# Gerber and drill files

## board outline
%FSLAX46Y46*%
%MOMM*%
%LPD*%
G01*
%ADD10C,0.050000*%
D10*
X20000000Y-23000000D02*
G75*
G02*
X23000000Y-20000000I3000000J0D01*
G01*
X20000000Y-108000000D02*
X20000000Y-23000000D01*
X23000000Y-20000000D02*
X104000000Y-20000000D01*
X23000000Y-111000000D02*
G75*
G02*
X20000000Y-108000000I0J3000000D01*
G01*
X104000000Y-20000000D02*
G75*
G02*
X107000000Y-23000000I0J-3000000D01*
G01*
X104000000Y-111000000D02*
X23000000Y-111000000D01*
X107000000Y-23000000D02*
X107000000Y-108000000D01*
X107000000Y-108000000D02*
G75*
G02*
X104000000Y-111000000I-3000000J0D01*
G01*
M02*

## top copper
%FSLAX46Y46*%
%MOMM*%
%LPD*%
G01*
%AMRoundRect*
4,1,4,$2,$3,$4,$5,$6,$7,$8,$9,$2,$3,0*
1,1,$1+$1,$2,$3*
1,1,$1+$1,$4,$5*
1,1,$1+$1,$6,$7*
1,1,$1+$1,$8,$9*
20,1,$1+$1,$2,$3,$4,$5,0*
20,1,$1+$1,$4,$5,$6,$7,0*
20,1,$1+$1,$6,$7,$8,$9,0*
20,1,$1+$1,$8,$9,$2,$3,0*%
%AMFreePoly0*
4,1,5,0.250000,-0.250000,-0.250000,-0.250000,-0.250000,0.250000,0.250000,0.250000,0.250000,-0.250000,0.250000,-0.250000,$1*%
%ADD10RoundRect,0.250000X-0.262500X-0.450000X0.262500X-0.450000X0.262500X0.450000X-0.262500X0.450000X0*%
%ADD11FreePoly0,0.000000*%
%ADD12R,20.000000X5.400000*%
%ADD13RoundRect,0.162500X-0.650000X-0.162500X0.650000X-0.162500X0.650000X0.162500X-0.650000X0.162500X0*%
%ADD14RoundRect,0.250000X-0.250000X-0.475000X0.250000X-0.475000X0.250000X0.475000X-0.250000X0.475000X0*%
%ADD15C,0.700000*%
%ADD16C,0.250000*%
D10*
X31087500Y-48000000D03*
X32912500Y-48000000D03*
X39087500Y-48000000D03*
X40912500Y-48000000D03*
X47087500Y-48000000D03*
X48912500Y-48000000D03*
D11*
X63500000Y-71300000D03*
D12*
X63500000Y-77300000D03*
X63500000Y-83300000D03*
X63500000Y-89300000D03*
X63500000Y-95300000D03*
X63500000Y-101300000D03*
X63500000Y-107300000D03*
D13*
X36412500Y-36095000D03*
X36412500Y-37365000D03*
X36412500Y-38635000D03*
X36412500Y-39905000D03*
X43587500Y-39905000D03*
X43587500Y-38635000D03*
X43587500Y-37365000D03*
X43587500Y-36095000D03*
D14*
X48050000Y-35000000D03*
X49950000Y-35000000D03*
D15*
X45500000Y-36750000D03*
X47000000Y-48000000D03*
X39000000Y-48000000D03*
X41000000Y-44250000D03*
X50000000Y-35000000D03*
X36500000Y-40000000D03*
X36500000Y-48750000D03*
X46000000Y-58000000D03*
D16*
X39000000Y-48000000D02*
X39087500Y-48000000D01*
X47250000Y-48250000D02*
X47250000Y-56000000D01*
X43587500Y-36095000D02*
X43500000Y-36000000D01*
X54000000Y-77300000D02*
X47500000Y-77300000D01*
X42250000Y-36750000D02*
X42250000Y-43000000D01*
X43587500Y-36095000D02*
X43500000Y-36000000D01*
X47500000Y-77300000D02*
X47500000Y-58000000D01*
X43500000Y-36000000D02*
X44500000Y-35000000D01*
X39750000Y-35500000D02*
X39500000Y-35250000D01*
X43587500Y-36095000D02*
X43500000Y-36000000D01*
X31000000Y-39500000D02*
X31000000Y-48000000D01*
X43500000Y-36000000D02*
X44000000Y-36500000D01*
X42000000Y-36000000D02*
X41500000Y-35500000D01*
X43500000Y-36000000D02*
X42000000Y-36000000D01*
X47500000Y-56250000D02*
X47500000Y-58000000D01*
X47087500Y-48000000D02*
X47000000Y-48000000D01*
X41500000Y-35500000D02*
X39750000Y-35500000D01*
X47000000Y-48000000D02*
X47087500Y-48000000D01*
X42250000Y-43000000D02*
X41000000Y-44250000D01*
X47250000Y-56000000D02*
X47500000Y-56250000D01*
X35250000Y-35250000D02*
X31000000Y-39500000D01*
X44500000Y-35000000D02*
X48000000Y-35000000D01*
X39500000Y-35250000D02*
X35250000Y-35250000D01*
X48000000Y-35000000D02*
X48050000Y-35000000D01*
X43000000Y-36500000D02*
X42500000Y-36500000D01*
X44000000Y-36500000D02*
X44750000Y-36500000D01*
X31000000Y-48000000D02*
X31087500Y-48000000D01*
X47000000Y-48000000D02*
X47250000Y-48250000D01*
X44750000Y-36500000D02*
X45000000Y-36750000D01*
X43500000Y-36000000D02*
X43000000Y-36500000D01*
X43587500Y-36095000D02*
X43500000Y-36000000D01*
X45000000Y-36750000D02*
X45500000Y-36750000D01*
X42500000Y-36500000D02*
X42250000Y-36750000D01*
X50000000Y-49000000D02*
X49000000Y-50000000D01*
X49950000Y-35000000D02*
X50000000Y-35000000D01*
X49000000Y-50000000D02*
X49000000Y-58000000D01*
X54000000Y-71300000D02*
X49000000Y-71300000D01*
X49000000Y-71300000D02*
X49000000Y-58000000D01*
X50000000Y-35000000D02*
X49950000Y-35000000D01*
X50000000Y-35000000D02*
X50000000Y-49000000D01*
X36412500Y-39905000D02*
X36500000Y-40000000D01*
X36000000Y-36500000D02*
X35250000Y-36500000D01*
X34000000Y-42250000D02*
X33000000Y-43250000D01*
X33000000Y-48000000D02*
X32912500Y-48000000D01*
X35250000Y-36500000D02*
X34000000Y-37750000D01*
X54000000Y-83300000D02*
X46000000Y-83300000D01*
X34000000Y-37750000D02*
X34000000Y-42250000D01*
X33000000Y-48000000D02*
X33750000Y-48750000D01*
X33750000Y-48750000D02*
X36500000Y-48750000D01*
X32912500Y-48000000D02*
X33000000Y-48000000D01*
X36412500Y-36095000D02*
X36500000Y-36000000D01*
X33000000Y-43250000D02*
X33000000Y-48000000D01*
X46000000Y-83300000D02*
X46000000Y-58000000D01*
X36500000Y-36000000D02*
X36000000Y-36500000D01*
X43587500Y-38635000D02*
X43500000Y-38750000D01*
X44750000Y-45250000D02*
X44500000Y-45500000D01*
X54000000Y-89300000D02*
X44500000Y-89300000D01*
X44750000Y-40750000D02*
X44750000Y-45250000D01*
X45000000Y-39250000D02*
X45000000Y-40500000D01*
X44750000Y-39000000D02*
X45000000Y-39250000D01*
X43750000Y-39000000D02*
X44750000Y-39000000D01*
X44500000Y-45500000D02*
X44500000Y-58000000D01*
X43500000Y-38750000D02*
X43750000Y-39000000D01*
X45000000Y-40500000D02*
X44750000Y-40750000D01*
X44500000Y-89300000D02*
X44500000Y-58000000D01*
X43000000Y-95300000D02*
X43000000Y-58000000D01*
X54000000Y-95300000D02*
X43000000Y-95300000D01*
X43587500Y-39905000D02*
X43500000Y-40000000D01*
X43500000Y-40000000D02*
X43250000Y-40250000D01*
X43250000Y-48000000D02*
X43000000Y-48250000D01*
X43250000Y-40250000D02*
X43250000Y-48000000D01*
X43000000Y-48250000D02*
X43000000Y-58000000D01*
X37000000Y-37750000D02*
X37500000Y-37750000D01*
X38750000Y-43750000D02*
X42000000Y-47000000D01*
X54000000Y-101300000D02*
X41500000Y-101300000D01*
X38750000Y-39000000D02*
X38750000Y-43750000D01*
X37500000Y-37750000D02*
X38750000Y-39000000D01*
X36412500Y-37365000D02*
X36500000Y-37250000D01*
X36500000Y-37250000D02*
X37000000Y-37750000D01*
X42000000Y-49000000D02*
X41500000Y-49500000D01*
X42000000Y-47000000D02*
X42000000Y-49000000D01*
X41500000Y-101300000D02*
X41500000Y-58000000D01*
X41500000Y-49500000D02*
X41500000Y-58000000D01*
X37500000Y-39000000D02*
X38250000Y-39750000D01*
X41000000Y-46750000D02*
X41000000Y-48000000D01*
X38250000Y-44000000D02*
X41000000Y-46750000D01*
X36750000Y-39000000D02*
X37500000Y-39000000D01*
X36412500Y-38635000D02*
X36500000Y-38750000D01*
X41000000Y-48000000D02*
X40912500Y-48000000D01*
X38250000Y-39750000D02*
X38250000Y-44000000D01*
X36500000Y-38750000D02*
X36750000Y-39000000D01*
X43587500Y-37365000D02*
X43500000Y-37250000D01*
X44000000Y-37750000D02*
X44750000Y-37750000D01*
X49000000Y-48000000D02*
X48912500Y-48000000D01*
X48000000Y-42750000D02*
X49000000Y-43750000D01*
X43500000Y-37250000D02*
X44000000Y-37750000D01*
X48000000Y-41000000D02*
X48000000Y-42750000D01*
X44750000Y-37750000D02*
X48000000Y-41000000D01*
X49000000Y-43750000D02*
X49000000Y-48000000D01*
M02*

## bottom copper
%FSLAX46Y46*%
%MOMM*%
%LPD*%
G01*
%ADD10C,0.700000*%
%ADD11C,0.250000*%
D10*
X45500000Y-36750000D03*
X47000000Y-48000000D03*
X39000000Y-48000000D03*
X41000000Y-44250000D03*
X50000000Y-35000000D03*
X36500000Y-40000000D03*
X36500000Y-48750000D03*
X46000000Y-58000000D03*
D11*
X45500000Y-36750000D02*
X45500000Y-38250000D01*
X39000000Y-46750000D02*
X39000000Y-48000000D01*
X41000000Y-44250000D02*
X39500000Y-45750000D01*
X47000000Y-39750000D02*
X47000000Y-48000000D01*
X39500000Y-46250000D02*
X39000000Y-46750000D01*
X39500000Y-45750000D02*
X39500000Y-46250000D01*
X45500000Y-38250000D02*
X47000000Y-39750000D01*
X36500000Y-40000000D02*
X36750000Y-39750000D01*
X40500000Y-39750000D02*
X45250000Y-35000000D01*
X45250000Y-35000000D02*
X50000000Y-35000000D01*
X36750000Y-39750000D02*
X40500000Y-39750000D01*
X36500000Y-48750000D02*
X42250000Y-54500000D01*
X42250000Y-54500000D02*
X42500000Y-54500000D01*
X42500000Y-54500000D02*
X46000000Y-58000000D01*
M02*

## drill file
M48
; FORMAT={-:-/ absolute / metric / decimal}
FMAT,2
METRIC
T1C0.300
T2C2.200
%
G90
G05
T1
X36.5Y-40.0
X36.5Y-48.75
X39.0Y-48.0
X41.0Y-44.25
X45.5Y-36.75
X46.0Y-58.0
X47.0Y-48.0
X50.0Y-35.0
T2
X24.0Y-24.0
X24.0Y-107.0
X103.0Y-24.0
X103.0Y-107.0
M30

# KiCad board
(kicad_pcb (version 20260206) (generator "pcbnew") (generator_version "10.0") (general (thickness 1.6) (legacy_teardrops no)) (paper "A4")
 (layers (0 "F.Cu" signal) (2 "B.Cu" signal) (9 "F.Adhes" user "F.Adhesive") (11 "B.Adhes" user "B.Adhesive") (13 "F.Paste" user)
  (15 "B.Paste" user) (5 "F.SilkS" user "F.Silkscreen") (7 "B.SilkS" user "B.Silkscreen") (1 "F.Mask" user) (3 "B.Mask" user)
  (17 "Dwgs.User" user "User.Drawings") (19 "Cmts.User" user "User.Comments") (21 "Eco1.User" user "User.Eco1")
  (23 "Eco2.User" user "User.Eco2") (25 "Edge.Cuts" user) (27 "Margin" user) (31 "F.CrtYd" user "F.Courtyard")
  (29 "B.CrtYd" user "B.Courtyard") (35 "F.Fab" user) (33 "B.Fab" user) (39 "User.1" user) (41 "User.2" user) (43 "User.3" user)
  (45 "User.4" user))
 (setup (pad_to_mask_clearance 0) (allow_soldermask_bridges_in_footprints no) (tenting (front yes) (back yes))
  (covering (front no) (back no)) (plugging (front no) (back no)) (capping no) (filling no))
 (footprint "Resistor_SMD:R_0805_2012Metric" (layer "F.Cu") (at 32 48)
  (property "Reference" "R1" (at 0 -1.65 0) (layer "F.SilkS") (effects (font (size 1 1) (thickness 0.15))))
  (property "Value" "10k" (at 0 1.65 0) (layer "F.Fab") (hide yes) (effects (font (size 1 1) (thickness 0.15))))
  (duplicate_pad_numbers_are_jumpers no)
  (pad "1" smd roundrect (at -0.9125 0) (size 1.025 1.4) (layers "F.Cu" "F.Mask" "F.Paste") (roundrect_rratio 0.243902) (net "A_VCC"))
  (pad "2" smd roundrect (at 0.9125 0) (size 1.025 1.4) (layers "F.Cu" "F.Mask" "F.Paste") (roundrect_rratio 0.243902) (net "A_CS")))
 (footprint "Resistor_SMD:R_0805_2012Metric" (layer "F.Cu") (at 40 48)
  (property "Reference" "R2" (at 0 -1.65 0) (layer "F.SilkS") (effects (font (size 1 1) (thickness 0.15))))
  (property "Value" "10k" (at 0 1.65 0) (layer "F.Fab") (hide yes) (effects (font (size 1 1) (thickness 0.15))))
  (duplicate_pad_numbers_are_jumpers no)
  (pad "1" smd roundrect (at -0.9125 0) (size 1.025 1.4) (layers "F.Cu" "F.Mask" "F.Paste") (roundrect_rratio 0.243902) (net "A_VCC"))
  (pad "2" smd roundrect (at 0.9125 0) (size 1.025 1.4) (layers "F.Cu" "F.Mask" "F.Paste") (roundrect_rratio 0.243902) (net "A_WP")))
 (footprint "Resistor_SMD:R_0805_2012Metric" (layer "F.Cu") (at 48 48)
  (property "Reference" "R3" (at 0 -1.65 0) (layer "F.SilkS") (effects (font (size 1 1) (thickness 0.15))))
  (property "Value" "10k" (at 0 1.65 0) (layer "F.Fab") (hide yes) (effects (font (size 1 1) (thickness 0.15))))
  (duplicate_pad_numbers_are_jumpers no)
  (pad "1" smd roundrect (at -0.9125 0) (size 1.025 1.4) (layers "F.Cu" "F.Mask" "F.Paste") (roundrect_rratio 0.243902) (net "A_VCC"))
  (pad "2" smd roundrect (at 0.9125 0) (size 1.025 1.4) (layers "F.Cu" "F.Mask" "F.Paste") (roundrect_rratio 0.243902) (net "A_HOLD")))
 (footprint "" (layer "F.Cu") (at 24 107)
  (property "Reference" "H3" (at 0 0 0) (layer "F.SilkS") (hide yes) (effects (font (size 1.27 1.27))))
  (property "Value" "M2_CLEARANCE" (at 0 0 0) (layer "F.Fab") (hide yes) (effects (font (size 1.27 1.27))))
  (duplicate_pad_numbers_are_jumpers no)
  (pad "" np_thru_hole circle (at 0 0) (size 2.2 2.2) (drill 2.2) (layers "*.Cu")))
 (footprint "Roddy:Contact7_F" (layer "F.Cu") (at 63.5 0)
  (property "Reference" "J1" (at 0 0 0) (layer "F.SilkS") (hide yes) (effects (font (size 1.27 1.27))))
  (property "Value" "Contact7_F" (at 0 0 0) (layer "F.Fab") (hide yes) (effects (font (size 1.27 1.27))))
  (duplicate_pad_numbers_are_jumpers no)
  (pad "1" smd custom (at 0 71.3) (size 0.5 0.5) (layers "F.Cu" "F.Mask") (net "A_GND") (solder_mask_margin 0.05) (thermal_bridge_angle 45)
   (options (clearance outline) (anchor rect)) (primitives))
  (pad "2" smd rect (at 0 77.3) (size 20 5.4) (layers "F.Cu" "F.Mask") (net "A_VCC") (solder_mask_margin 0.05) (thermal_bridge_angle 45))
  (pad "3" smd rect (at 0 83.3) (size 20 5.4) (layers "F.Cu" "F.Mask") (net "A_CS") (solder_mask_margin 0.05) (thermal_bridge_angle 45))
  (pad "4" smd rect (at 0 89.3) (size 20 5.4) (layers "F.Cu" "F.Mask") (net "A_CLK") (solder_mask_margin 0.05) (thermal_bridge_angle 45))
  (pad "5" smd rect (at 0 95.3) (size 20 5.4) (layers "F.Cu" "F.Mask") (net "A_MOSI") (solder_mask_margin 0.05) (thermal_bridge_angle 45))
  (pad "6" smd rect (at 0 101.3) (size 20 5.4) (layers "F.Cu" "F.Mask") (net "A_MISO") (solder_mask_margin 0.05) (thermal_bridge_angle 45))
  (pad "7" smd rect (at 0 107.3) (size 20 5.4) (layers "F.Cu" "F.Mask") (solder_mask_margin 0.05) (thermal_bridge_angle 45)))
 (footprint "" (layer "F.Cu") (at 24 24)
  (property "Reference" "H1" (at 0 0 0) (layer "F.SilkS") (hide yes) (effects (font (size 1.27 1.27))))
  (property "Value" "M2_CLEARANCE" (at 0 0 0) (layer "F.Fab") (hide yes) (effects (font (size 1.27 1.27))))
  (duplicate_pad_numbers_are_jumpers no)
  (pad "" np_thru_hole circle (at 0 0) (size 2.2 2.2) (drill 2.2) (layers "*.Cu")))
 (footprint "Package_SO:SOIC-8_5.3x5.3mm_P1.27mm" (layer "F.Cu") (at 40 38)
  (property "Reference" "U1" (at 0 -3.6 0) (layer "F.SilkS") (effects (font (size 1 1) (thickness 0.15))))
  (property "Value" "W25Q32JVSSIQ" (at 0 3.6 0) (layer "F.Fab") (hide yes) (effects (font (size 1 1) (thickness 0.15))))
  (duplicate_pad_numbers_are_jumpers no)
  (pad "1" smd roundrect (at -3.5875 -1.905) (size 1.625 0.65) (layers "F.Cu" "F.Mask" "F.Paste") (roundrect_rratio 0.25) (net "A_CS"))
  (pad "2" smd roundrect (at -3.5875 -0.635) (size 1.625 0.65) (layers "F.Cu" "F.Mask" "F.Paste") (roundrect_rratio 0.25) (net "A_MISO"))
  (pad "3" smd roundrect (at -3.5875 0.635) (size 1.625 0.65) (layers "F.Cu" "F.Mask" "F.Paste") (roundrect_rratio 0.25) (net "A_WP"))
  (pad "4" smd roundrect (at -3.5875 1.905) (size 1.625 0.65) (layers "F.Cu" "F.Mask" "F.Paste") (roundrect_rratio 0.25) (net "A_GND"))
  (pad "5" smd roundrect (at 3.5875 1.905) (size 1.625 0.65) (layers "F.Cu" "F.Mask" "F.Paste") (roundrect_rratio 0.25) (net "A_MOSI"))
  (pad "6" smd roundrect (at 3.5875 0.635) (size 1.625 0.65) (layers "F.Cu" "F.Mask" "F.Paste") (roundrect_rratio 0.25) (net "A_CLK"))
  (pad "7" smd roundrect (at 3.5875 -0.635) (size 1.625 0.65) (layers "F.Cu" "F.Mask" "F.Paste") (roundrect_rratio 0.25) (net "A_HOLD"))
  (pad "8" smd roundrect (at 3.5875 -1.905) (size 1.625 0.65) (layers "F.Cu" "F.Mask" "F.Paste") (roundrect_rratio 0.25) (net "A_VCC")))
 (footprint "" (layer "F.Cu") (at 103 107)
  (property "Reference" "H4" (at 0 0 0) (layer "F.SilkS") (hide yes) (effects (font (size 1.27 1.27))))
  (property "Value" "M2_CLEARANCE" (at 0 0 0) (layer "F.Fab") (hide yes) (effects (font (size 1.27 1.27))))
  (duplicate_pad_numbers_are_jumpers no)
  (pad "" np_thru_hole circle (at 0 0) (size 2.2 2.2) (drill 2.2) (layers "*.Cu")))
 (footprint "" (layer "F.Cu") (at 103 24)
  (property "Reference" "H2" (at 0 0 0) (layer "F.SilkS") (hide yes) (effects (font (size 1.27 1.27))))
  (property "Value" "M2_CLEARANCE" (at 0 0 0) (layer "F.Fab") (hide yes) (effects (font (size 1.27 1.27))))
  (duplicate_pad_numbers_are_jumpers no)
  (pad "" np_thru_hole circle (at 0 0) (size 2.2 2.2) (drill 2.2) (layers "*.Cu")))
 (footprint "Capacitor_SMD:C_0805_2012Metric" (layer "F.Cu") (at 49 35)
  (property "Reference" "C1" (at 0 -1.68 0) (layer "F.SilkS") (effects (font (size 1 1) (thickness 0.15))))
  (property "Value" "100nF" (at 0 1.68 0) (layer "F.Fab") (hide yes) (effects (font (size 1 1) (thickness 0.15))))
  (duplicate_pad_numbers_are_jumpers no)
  (pad "1" smd roundrect (at -0.95 0) (size 1 1.45) (layers "F.Cu" "F.Mask" "F.Paste") (roundrect_rratio 0.25) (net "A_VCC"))
  (pad "2" smd roundrect (at 0.95 0) (size 1 1.45) (layers "F.Cu" "F.Mask" "F.Paste") (roundrect_rratio 0.25) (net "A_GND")))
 (gr_arc (start 20 23) (mid 20.878679 20.878679) (end 23 20) (stroke (width 0.05) (type default)) (layer "Edge.Cuts"))
 (gr_line (start 20 108) (end 20 23) (stroke (width 0.05) (type default)) (layer "Edge.Cuts"))
 (gr_line (start 23 20) (end 104 20) (stroke (width 0.05) (type default)) (layer "Edge.Cuts"))
 (gr_arc (start 23 111) (mid 20.878679 110.12132) (end 20 108) (stroke (width 0.05) (type default)) (layer "Edge.Cuts"))
 (gr_arc (start 104 20) (mid 106.12132 20.878679) (end 107 23) (stroke (width 0.05) (type default)) (layer "Edge.Cuts"))
 (gr_line (start 104 111) (end 23 111) (stroke (width 0.05) (type default)) (layer "Edge.Cuts"))
 (gr_line (start 107 23) (end 107 108) (stroke (width 0.05) (type default)) (layer "Edge.Cuts"))
 (gr_arc (start 107 108) (mid 106.12132 110.12132) (end 104 111) (stroke (width 0.05) (type default)) (layer "Edge.Cuts"))
 (segment (start 39 48) (end 39.0875 48) (width 0.25) (layer "F.Cu") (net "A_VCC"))
 (segment (start 47.25 48.25) (end 47.25 56) (width 0.25) (layer "F.Cu") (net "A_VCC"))
 (segment (start 43.5875 36.095) (end 43.5 36) (width 0.25) (layer "F.Cu") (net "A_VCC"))
 (segment (start 54 77.3) (end 47.5 77.3) (width 0.25) (layer "F.Cu") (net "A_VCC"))
 (segment (start 42.25 36.75) (end 42.25 43) (width 0.25) (layer "F.Cu") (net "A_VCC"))
 (segment (start 43.5875 36.095) (end 43.5 36) (width 0.25) (layer "F.Cu") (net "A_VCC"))
 (segment (start 47.5 77.3) (end 47.5 58) (width 0.25) (layer "F.Cu") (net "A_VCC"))
 (segment (start 43.5 36) (end 44.5 35) (width 0.25) (layer "F.Cu") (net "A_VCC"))
 (segment (start 39.75 35.5) (end 39.5 35.25) (width 0.25) (layer "F.Cu") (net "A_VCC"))
 (segment (start 43.5875 36.095) (end 43.5 36) (width 0.25) (layer "F.Cu") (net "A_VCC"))
 (segment (start 31 39.5) (end 31 48) (width 0.25) (layer "F.Cu") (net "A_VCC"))
 (segment (start 43.5 36) (end 44 36.5) (width 0.25) (layer "F.Cu") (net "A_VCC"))
 (segment (start 42 36) (end 41.5 35.5) (width 0.25) (layer "F.Cu") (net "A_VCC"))
 (segment (start 43.5 36) (end 42 36) (width 0.25) (layer "F.Cu") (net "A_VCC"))
 (segment (start 47.5 56.25) (end 47.5 58) (width 0.25) (layer "F.Cu") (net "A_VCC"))
 (segment (start 47.0875 48) (end 47 48) (width 0.25) (layer "F.Cu") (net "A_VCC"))
 (segment (start 41.5 35.5) (end 39.75 35.5) (width 0.25) (layer "F.Cu") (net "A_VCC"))
 (segment (start 47 48) (end 47.0875 48) (width 0.25) (layer "F.Cu") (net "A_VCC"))
 (segment (start 42.25 43) (end 41 44.25) (width 0.25) (layer "F.Cu") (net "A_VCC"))
 (segment (start 47.25 56) (end 47.5 56.25) (width 0.25) (layer "F.Cu") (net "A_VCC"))
 (segment (start 35.25 35.25) (end 31 39.5) (width 0.25) (layer "F.Cu") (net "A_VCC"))
 (segment (start 44.5 35) (end 48 35) (width 0.25) (layer "F.Cu") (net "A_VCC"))
 (segment (start 39.5 35.25) (end 35.25 35.25) (width 0.25) (layer "F.Cu") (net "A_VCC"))
 (segment (start 48 35) (end 48.05 35) (width 0.25) (layer "F.Cu") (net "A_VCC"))
 (segment (start 43 36.5) (end 42.5 36.5) (width 0.25) (layer "F.Cu") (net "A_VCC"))
 (segment (start 44 36.5) (end 44.75 36.5) (width 0.25) (layer "F.Cu") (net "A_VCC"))
 (segment (start 31 48) (end 31.0875 48) (width 0.25) (layer "F.Cu") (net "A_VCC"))
 (segment (start 47 48) (end 47.25 48.25) (width 0.25) (layer "F.Cu") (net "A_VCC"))
 (segment (start 44.75 36.5) (end 45 36.75) (width 0.25) (layer "F.Cu") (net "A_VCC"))
 (segment (start 43.5 36) (end 43 36.5) (width 0.25) (layer "F.Cu") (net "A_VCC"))
 (segment (start 43.5875 36.095) (end 43.5 36) (width 0.25) (layer "F.Cu") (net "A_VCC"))
 (segment (start 45 36.75) (end 45.5 36.75) (width 0.25) (layer "F.Cu") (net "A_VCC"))
 (segment (start 42.5 36.5) (end 42.25 36.75) (width 0.25) (layer "F.Cu") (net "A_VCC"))
 (via (at 45.5 36.75) (size 0.7) (drill 0.3) (layers "F.Cu" "B.Cu") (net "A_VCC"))
 (via (at 47 48) (size 0.7) (drill 0.3) (layers "F.Cu" "B.Cu") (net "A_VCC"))
 (via (at 39 48) (size 0.7) (drill 0.3) (layers "F.Cu" "B.Cu") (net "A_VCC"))
 (via (at 41 44.25) (size 0.7) (drill 0.3) (layers "F.Cu" "B.Cu") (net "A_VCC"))
 (segment (start 45.5 36.75) (end 45.5 38.25) (width 0.25) (layer "B.Cu") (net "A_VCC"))
 (segment (start 39 46.75) (end 39 48) (width 0.25) (layer "B.Cu") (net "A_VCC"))
 (segment (start 41 44.25) (end 39.5 45.75) (width 0.25) (layer "B.Cu") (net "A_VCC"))
 (segment (start 47 39.75) (end 47 48) (width 0.25) (layer "B.Cu") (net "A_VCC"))
 (segment (start 39.5 46.25) (end 39 46.75) (width 0.25) (layer "B.Cu") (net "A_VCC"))
 (segment (start 39.5 45.75) (end 39.5 46.25) (width 0.25) (layer "B.Cu") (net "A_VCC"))
 (segment (start 45.5 38.25) (end 47 39.75) (width 0.25) (layer "B.Cu") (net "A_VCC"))
 (segment (start 50 49) (end 49 50) (width 0.25) (layer "F.Cu") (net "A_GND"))
 (segment (start 49.95 35) (end 50 35) (width 0.25) (layer "F.Cu") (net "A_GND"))
 (segment (start 49 50) (end 49 58) (width 0.25) (layer "F.Cu") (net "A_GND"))
 (segment (start 54 71.3) (end 49 71.3) (width 0.25) (layer "F.Cu") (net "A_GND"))
 (segment (start 49 71.3) (end 49 58) (width 0.25) (layer "F.Cu") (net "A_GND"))
 (segment (start 50 35) (end 49.95 35) (width 0.25) (layer "F.Cu") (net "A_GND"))
 (segment (start 50 35) (end 50 49) (width 0.25) (layer "F.Cu") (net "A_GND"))
 (segment (start 36.4125 39.905) (end 36.5 40) (width 0.25) (layer "F.Cu") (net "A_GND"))
 (via (at 50 35) (size 0.7) (drill 0.3) (layers "F.Cu" "B.Cu") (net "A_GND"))
 (via (at 36.5 40) (size 0.7) (drill 0.3) (layers "F.Cu" "B.Cu") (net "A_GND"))
 (segment (start 36.5 40) (end 36.75 39.75) (width 0.25) (layer "B.Cu") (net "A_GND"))
 (segment (start 40.5 39.75) (end 45.25 35) (width 0.25) (layer "B.Cu") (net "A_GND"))
 (segment (start 45.25 35) (end 50 35) (width 0.25) (layer "B.Cu") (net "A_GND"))
 (segment (start 36.75 39.75) (end 40.5 39.75) (width 0.25) (layer "B.Cu") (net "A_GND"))
 (segment (start 36 36.5) (end 35.25 36.5) (width 0.25) (layer "F.Cu") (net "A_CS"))
 (segment (start 34 42.25) (end 33 43.25) (width 0.25) (layer "F.Cu") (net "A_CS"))
 (segment (start 33 48) (end 32.9125 48) (width 0.25) (layer "F.Cu") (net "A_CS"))
 (segment (start 35.25 36.5) (end 34 37.75) (width 0.25) (layer "F.Cu") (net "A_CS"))
 (segment (start 54 83.3) (end 46 83.3) (width 0.25) (layer "F.Cu") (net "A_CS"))
 (segment (start 34 37.75) (end 34 42.25) (width 0.25) (layer "F.Cu") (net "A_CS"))
 (segment (start 33 48) (end 33.75 48.75) (width 0.25) (layer "F.Cu") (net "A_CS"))
 (segment (start 33.75 48.75) (end 36.5 48.75) (width 0.25) (layer "F.Cu") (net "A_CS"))
 (segment (start 32.9125 48) (end 33 48) (width 0.25) (layer "F.Cu") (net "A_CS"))
 (segment (start 36.4125 36.095) (end 36.5 36) (width 0.25) (layer "F.Cu") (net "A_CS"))
 (segment (start 33 43.25) (end 33 48) (width 0.25) (layer "F.Cu") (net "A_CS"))
 (segment (start 46 83.3) (end 46 58) (width 0.25) (layer "F.Cu") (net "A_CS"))
 (segment (start 36.5 36) (end 36 36.5) (width 0.25) (layer "F.Cu") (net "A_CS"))
 (via (at 36.5 48.75) (size 0.7) (drill 0.3) (layers "F.Cu" "B.Cu") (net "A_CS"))
 (via (at 46 58) (size 0.7) (drill 0.3) (layers "F.Cu" "B.Cu") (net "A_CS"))
 (segment (start 36.5 48.75) (end 42.25 54.5) (width 0.25) (layer "B.Cu") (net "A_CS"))
 (segment (start 42.25 54.5) (end 42.5 54.5) (width 0.25) (layer "B.Cu") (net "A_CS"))
 (segment (start 42.5 54.5) (end 46 58) (width 0.25) (layer "B.Cu") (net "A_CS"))
 (segment (start 43.5875 38.635) (end 43.5 38.75) (width 0.25) (layer "F.Cu") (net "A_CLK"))
 (segment (start 44.75 45.25) (end 44.5 45.5) (width 0.25) (layer "F.Cu") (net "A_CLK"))
 (segment (start 54 89.3) (end 44.5 89.3) (width 0.25) (layer "F.Cu") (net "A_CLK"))
 (segment (start 44.75 40.75) (end 44.75 45.25) (width 0.25) (layer "F.Cu") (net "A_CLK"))
 (segment (start 45 39.25) (end 45 40.5) (width 0.25) (layer "F.Cu") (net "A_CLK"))
 (segment (start 44.75 39) (end 45 39.25) (width 0.25) (layer "F.Cu") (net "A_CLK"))
 (segment (start 43.75 39) (end 44.75 39) (width 0.25) (layer "F.Cu") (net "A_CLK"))
 (segment (start 44.5 45.5) (end 44.5 58) (width 0.25) (layer "F.Cu") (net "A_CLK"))
 (segment (start 43.5 38.75) (end 43.75 39) (width 0.25) (layer "F.Cu") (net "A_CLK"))
 (segment (start 45 40.5) (end 44.75 40.75) (width 0.25) (layer "F.Cu") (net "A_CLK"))
 (segment (start 44.5 89.3) (end 44.5 58) (width 0.25) (layer "F.Cu") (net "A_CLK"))
 (segment (start 43 95.3) (end 43 58) (width 0.25) (layer "F.Cu") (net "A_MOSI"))
 (segment (start 54 95.3) (end 43 95.3) (width 0.25) (layer "F.Cu") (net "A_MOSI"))
 (segment (start 43.5875 39.905) (end 43.5 40) (width 0.25) (layer "F.Cu") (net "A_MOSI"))
 (segment (start 43.5 40) (end 43.25 40.25) (width 0.25) (layer "F.Cu") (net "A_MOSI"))
 (segment (start 43.25 48) (end 43 48.25) (width 0.25) (layer "F.Cu") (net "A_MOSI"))
 (segment (start 43.25 40.25) (end 43.25 48) (width 0.25) (layer "F.Cu") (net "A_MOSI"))
 (segment (start 43 48.25) (end 43 58) (width 0.25) (layer "F.Cu") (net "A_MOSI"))
 (segment (start 37 37.75) (end 37.5 37.75) (width 0.25) (layer "F.Cu") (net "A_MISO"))
 (segment (start 38.75 43.75) (end 42 47) (width 0.25) (layer "F.Cu") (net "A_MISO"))
 (segment (start 54 101.3) (end 41.5 101.3) (width 0.25) (layer "F.Cu") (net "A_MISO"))
 (segment (start 38.75 39) (end 38.75 43.75) (width 0.25) (layer "F.Cu") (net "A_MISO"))
 (segment (start 37.5 37.75) (end 38.75 39) (width 0.25) (layer "F.Cu") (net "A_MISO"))
 (segment (start 36.4125 37.365) (end 36.5 37.25) (width 0.25) (layer "F.Cu") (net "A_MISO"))
 (segment (start 36.5 37.25) (end 37 37.75) (width 0.25) (layer "F.Cu") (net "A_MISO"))
 (segment (start 42 49) (end 41.5 49.5) (width 0.25) (layer "F.Cu") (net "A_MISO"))
 (segment (start 42 47) (end 42 49) (width 0.25) (layer "F.Cu") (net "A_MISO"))
 (segment (start 41.5 101.3) (end 41.5 58) (width 0.25) (layer "F.Cu") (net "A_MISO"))
 (segment (start 41.5 49.5) (end 41.5 58) (width 0.25) (layer "F.Cu") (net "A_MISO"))
 (segment (start 37.5 39) (end 38.25 39.75) (width 0.25) (layer "F.Cu") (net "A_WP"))
 (segment (start 41 46.75) (end 41 48) (width 0.25) (layer "F.Cu") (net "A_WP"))
 (segment (start 38.25 44) (end 41 46.75) (width 0.25) (layer "F.Cu") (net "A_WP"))
 (segment (start 36.75 39) (end 37.5 39) (width 0.25) (layer "F.Cu") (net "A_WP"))
 (segment (start 36.4125 38.635) (end 36.5 38.75) (width 0.25) (layer "F.Cu") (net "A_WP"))
 (segment (start 41 48) (end 40.9125 48) (width 0.25) (layer "F.Cu") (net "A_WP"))
 (segment (start 38.25 39.75) (end 38.25 44) (width 0.25) (layer "F.Cu") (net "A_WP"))
 (segment (start 36.5 38.75) (end 36.75 39) (width 0.25) (layer "F.Cu") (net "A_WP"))
 (segment (start 43.5875 37.365) (end 43.5 37.25) (width 0.25) (layer "F.Cu") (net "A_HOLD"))
 (segment (start 44 37.75) (end 44.75 37.75) (width 0.25) (layer "F.Cu") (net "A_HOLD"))
 (segment (start 49 48) (end 48.9125 48) (width 0.25) (layer "F.Cu") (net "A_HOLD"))
 (segment (start 48 42.75) (end 49 43.75) (width 0.25) (layer "F.Cu") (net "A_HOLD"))
 (segment (start 43.5 37.25) (end 44 37.75) (width 0.25) (layer "F.Cu") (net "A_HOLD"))
 (segment (start 48 41) (end 48 42.75) (width 0.25) (layer "F.Cu") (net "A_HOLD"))
 (segment (start 44.75 37.75) (end 48 41) (width 0.25) (layer "F.Cu") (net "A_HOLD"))
 (segment (start 49 43.75) (end 49 48) (width 0.25) (layer "F.Cu") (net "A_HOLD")))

